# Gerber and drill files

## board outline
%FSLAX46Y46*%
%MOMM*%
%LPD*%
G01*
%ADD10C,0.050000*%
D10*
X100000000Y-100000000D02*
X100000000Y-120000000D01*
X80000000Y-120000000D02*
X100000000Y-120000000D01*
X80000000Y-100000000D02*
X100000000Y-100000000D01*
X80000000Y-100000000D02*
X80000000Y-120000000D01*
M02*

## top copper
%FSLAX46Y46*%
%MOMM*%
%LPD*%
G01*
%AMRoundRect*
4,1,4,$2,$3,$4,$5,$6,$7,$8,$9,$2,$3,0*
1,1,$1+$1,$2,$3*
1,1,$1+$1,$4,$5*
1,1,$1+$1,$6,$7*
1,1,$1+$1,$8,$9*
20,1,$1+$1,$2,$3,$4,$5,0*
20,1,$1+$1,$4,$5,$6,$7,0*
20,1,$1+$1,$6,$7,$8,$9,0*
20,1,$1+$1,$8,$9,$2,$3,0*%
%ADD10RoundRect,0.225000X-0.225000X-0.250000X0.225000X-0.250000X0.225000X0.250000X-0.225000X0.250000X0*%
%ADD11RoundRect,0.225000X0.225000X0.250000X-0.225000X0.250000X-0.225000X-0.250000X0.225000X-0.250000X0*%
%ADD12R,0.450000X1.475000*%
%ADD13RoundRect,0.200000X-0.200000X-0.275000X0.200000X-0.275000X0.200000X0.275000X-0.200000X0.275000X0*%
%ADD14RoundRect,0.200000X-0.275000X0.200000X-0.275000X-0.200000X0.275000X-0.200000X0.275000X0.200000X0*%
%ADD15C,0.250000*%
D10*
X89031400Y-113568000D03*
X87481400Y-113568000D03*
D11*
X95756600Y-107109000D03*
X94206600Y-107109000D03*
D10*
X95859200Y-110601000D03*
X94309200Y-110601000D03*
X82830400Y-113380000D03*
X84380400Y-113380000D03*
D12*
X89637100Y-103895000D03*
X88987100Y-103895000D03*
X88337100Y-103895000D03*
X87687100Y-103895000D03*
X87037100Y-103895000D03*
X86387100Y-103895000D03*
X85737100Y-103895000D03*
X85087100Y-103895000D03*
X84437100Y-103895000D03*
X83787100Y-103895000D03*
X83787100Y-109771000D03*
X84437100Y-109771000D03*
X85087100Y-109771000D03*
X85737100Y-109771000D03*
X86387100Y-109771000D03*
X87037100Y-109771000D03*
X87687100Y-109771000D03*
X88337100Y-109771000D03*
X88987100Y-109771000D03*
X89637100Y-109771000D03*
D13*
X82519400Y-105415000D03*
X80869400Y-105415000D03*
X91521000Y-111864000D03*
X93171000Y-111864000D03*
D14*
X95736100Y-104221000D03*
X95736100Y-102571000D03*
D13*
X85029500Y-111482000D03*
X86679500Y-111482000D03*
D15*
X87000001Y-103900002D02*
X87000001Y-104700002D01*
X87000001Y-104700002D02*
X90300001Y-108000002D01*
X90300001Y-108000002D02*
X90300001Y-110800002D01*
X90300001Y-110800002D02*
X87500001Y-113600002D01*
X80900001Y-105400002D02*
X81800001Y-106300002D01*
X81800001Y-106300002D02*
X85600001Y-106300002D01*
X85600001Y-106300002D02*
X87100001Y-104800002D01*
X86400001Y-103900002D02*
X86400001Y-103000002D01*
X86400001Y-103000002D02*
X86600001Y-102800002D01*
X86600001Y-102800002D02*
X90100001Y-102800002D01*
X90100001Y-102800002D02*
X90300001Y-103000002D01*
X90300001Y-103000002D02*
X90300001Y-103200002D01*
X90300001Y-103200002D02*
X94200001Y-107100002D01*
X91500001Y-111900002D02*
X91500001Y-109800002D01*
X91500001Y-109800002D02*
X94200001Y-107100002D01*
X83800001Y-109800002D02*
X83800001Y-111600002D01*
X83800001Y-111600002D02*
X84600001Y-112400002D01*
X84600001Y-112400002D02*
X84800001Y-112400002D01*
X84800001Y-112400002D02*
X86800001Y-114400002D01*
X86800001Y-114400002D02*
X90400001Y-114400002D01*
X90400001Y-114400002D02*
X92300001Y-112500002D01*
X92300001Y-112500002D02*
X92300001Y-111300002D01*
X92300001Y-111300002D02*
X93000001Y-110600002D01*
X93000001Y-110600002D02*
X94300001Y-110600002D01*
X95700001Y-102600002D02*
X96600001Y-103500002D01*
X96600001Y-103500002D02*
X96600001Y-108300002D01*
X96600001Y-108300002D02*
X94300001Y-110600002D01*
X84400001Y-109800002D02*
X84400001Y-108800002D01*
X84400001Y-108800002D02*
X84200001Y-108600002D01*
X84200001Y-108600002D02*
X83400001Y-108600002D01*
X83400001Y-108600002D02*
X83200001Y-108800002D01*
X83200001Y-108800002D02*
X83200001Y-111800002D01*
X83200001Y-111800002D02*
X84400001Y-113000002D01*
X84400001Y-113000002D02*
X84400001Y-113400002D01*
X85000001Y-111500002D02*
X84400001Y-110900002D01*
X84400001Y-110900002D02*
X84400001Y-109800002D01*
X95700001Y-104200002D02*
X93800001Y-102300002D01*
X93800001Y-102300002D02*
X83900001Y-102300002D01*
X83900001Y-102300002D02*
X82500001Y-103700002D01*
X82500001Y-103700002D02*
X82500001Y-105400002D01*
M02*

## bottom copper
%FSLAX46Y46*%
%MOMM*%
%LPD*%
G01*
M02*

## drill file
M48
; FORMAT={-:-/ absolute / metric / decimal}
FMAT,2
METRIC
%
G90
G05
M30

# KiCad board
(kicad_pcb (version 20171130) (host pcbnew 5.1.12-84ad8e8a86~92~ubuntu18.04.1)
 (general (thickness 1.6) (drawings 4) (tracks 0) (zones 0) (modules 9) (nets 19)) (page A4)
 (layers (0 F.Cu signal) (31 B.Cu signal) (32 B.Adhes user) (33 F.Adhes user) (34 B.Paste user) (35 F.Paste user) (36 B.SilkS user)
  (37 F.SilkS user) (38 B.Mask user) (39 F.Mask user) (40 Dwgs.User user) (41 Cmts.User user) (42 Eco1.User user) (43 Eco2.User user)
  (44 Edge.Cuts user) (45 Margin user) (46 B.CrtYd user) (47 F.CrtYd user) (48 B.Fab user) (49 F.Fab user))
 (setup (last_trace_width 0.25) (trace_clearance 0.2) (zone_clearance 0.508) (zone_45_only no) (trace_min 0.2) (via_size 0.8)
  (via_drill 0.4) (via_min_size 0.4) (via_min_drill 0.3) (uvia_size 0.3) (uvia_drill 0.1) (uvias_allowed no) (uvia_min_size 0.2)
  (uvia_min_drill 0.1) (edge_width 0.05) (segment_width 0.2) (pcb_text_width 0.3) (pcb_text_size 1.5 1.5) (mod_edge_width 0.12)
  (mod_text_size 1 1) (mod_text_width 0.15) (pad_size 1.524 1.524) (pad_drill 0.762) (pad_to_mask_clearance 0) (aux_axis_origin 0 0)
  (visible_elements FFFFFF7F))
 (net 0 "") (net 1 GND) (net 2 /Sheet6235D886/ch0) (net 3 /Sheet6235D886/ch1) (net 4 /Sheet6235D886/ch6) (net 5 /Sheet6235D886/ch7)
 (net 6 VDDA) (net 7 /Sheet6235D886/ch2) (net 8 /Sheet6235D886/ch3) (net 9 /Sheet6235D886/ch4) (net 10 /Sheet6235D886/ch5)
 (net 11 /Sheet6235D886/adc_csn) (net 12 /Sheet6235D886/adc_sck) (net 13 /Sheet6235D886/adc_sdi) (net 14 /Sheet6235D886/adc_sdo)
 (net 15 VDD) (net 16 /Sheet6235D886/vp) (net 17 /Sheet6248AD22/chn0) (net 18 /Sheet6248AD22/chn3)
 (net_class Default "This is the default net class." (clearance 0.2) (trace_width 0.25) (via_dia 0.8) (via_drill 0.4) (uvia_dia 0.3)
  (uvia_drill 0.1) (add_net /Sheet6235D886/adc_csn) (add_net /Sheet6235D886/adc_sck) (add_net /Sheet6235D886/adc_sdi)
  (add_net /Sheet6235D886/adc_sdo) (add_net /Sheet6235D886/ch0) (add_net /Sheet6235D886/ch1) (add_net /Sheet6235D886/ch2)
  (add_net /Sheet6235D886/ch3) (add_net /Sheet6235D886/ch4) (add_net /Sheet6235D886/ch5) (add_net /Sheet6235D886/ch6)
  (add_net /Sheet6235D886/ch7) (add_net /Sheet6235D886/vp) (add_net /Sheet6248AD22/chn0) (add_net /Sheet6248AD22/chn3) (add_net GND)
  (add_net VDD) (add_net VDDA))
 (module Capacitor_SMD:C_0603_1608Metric (layer F.Cu) (at 88.256400 113.568000)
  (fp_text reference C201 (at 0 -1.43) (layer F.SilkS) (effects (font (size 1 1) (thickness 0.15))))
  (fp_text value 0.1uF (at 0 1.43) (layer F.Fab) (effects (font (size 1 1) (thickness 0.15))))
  (pad 2 smd roundrect (at 0.775 0) (size 0.9 0.95) (layers F.Cu F.Mask F.Paste) (roundrect_rratio 0.25) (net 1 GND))
  (pad 1 smd roundrect (at -0.775 0) (size 0.9 0.95) (layers F.Cu F.Mask F.Paste) (roundrect_rratio 0.25) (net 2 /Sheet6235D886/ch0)))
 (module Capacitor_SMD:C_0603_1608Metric (layer F.Cu) (at 94.981600 107.109000 180.000000)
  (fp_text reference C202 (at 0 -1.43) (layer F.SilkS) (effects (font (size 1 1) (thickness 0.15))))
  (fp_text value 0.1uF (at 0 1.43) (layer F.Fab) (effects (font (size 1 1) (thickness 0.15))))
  (pad 1 smd roundrect (at -0.775 0 180.000000) (size 0.9 0.95) (layers F.Cu F.Mask F.Paste) (roundrect_rratio 0.25) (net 1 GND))
  (pad 2 smd roundrect (at 0.775 0 180.000000) (size 0.9 0.95) (layers F.Cu F.Mask F.Paste) (roundrect_rratio 0.25)
   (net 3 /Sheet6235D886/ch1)))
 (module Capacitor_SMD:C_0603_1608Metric (layer F.Cu) (at 95.084200 110.601000)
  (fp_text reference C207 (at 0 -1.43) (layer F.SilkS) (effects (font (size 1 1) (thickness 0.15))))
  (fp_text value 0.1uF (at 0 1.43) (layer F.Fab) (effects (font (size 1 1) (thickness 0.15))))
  (pad 2 smd roundrect (at 0.775 0) (size 0.9 0.95) (layers F.Cu F.Mask F.Paste) (roundrect_rratio 0.25) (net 1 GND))
  (pad 1 smd roundrect (at -0.775 0) (size 0.9 0.95) (layers F.Cu F.Mask F.Paste) (roundrect_rratio 0.25) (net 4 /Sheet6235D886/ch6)))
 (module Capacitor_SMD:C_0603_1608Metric (layer F.Cu) (at 83.605400 113.380000)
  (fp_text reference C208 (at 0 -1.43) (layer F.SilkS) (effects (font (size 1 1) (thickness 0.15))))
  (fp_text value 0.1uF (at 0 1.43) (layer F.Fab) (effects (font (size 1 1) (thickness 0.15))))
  (pad 1 smd roundrect (at -0.775 0) (size 0.9 0.95) (layers F.Cu F.Mask F.Paste) (roundrect_rratio 0.25) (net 1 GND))
  (pad 2 smd roundrect (at 0.775 0) (size 0.9 0.95) (layers F.Cu F.Mask F.Paste) (roundrect_rratio 0.25) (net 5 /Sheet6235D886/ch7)))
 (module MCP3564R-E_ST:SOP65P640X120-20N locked (layer F.Cu) (at 86.712100 106.833000 270.000000)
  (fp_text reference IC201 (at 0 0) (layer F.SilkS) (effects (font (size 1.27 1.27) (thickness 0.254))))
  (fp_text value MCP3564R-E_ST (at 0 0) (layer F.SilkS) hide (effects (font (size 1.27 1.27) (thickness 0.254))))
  (pad 1 smd rect (at -2.938 -2.925) (size 0.45 1.475) (layers F.Cu F.Mask F.Paste) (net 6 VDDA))
  (pad 2 smd rect (at -2.938 -2.275) (size 0.45 1.475) (layers F.Cu F.Mask F.Paste) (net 1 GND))
  (pad 3 smd rect (at -2.938 -1.625) (size 0.45 1.475) (layers F.Cu F.Mask F.Paste) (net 1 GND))
  (pad 4 smd rect (at -2.938 -0.975) (size 0.45 1.475) (layers F.Cu F.Mask F.Paste))
  (pad 5 smd rect (at -2.938 -0.325) (size 0.45 1.475) (layers F.Cu F.Mask F.Paste) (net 2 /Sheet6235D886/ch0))
  (pad 6 smd rect (at -2.938 0.325) (size 0.45 1.475) (layers F.Cu F.Mask F.Paste) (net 3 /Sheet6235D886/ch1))
  (pad 7 smd rect (at -2.938 0.975) (size 0.45 1.475) (layers F.Cu F.Mask F.Paste) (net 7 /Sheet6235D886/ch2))
  (pad 8 smd rect (at -2.938 1.625) (size 0.45 1.475) (layers F.Cu F.Mask F.Paste) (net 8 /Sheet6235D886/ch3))
  (pad 9 smd rect (at -2.938 2.275) (size 0.45 1.475) (layers F.Cu F.Mask F.Paste) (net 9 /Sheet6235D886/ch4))
  (pad 10 smd rect (at -2.938 2.925) (size 0.45 1.475) (layers F.Cu F.Mask F.Paste) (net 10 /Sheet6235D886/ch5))
  (pad 11 smd rect (at 2.938 2.925) (size 0.45 1.475) (layers F.Cu F.Mask F.Paste) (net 4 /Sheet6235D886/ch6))
  (pad 12 smd rect (at 2.938 2.275) (size 0.45 1.475) (layers F.Cu F.Mask F.Paste) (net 5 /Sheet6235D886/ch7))
  (pad 13 smd rect (at 2.938 1.625) (size 0.45 1.475) (layers F.Cu F.Mask F.Paste) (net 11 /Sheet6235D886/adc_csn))
  (pad 14 smd rect (at 2.938 0.975) (size 0.45 1.475) (layers F.Cu F.Mask F.Paste) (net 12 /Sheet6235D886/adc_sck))
  (pad 15 smd rect (at 2.938 0.325) (size 0.45 1.475) (layers F.Cu F.Mask F.Paste) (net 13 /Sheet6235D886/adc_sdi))
  (pad 16 smd rect (at 2.938 -0.325) (size 0.45 1.475) (layers F.Cu F.Mask F.Paste) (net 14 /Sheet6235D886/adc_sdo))
  (pad 17 smd rect (at 2.938 -0.975) (size 0.45 1.475) (layers F.Cu F.Mask F.Paste))
  (pad 18 smd rect (at 2.938 -1.625) (size 0.45 1.475) (layers F.Cu F.Mask F.Paste))
  (pad 19 smd rect (at 2.938 -2.275) (size 0.45 1.475) (layers F.Cu F.Mask F.Paste) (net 1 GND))
  (pad 20 smd rect (at 2.938 -2.925) (size 0.45 1.475) (layers F.Cu F.Mask F.Paste) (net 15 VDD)))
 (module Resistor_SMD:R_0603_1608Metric (layer F.Cu) (at 81.694400 105.415000)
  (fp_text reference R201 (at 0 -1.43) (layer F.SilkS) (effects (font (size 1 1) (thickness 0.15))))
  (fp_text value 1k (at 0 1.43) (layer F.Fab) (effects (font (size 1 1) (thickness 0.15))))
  (pad 2 smd roundrect (at 0.825 0) (size 0.8 0.95) (layers F.Cu F.Mask F.Paste) (roundrect_rratio 0.25) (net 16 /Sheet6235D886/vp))
  (pad 1 smd roundrect (at -0.825 0) (size 0.8 0.95) (layers F.Cu F.Mask F.Paste) (roundrect_rratio 0.25) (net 2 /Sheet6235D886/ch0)))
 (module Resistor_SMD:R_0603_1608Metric (layer F.Cu) (at 92.346000 111.864000)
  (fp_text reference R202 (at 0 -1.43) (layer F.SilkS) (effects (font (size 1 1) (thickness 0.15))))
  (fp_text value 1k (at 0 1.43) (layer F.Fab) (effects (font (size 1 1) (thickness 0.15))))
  (pad 1 smd roundrect (at -0.825 0) (size 0.8 0.95) (layers F.Cu F.Mask F.Paste) (roundrect_rratio 0.25) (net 3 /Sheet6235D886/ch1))
  (pad 2 smd roundrect (at 0.825 0) (size 0.8 0.95) (layers F.Cu F.Mask F.Paste) (roundrect_rratio 0.25) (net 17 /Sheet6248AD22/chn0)))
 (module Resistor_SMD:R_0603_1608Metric (layer F.Cu) (at 95.736100 103.396000 270.000000)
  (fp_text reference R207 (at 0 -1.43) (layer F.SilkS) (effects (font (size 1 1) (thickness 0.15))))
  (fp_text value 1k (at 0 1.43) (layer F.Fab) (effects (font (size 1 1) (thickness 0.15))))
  (pad 2 smd roundrect (at 0.825 0 270.000000) (size 0.8 0.95) (layers F.Cu F.Mask F.Paste) (roundrect_rratio 0.25)
   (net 16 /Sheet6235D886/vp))
  (pad 1 smd roundrect (at -0.825 0 270.000000) (size 0.8 0.95) (layers F.Cu F.Mask F.Paste) (roundrect_rratio 0.25)
   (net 4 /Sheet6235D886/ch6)))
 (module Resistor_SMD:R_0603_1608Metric (layer F.Cu) (at 85.854500 111.482000)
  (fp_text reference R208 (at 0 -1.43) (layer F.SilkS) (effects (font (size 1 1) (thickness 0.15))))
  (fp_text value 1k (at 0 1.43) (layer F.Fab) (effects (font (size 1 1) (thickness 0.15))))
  (pad 1 smd roundrect (at -0.825 0) (size 0.8 0.95) (layers F.Cu F.Mask F.Paste) (roundrect_rratio 0.25) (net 5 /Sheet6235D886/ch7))
  (pad 2 smd roundrect (at 0.825 0) (size 0.8 0.95) (layers F.Cu F.Mask F.Paste) (roundrect_rratio 0.25) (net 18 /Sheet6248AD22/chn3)))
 (gr_line (start 100 100) (end 100 120) (layer Edge.Cuts) (width 0.05))
 (gr_line (start 80 120) (end 100 120) (layer Edge.Cuts) (width 0.05))
 (gr_line (start 80 100) (end 100 100) (layer Edge.Cuts) (width 0.05))
 (gr_line (start 80 100) (end 80 120) (layer Edge.Cuts) (width 0.05))
 (segment (start 87.000001 103.900002) (end 87.000001 104.700002) (width 0.250000) (layer F.Cu) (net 2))
 (segment (start 87.000001 104.700002) (end 90.300001 108.000002) (width 0.250000) (layer F.Cu) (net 2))
 (segment (start 90.300001 108.000002) (end 90.300001 110.800002) (width 0.250000) (layer F.Cu) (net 2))
 (segment (start 90.300001 110.800002) (end 87.500001 113.600002) (width 0.250000) (layer F.Cu) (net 2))
 (segment (start 80.900001 105.400002) (end 81.800001 106.300002) (width 0.250000) (layer F.Cu) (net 2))
 (segment (start 81.800001 106.300002) (end 85.600001 106.300002) (width 0.250000) (layer F.Cu) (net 2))
 (segment (start 85.600001 106.300002) (end 87.100001 104.800002) (width 0.250000) (layer F.Cu) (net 2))
 (segment (start 86.400001 103.900002) (end 86.400001 103.000002) (width 0.250000) (layer F.Cu) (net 3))
 (segment (start 86.400001 103.000002) (end 86.600001 102.800002) (width 0.250000) (layer F.Cu) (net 3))
 (segment (start 86.600001 102.800002) (end 90.100001 102.800002) (width 0.250000) (layer F.Cu) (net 3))
 (segment (start 90.100001 102.800002) (end 90.300001 103.000002) (width 0.250000) (layer F.Cu) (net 3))
 (segment (start 90.300001 103.000002) (end 90.300001 103.200002) (width 0.250000) (layer F.Cu) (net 3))
 (segment (start 90.300001 103.200002) (end 94.200001 107.100002) (width 0.250000) (layer F.Cu) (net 3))
 (segment (start 91.500001 111.900002) (end 91.500001 109.800002) (width 0.250000) (layer F.Cu) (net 3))
 (segment (start 91.500001 109.800002) (end 94.200001 107.100002) (width 0.250000) (layer F.Cu) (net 3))
 (segment (start 83.800001 109.800002) (end 83.800001 111.600002) (width 0.250000) (layer F.Cu) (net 4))
 (segment (start 83.800001 111.600002) (end 84.600001 112.400002) (width 0.250000) (layer F.Cu) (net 4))
 (segment (start 84.600001 112.400002) (end 84.800001 112.400002) (width 0.250000) (layer F.Cu) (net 4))
 (segment (start 84.800001 112.400002) (end 86.800001 114.400002) (width 0.250000) (layer F.Cu) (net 4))
 (segment (start 86.800001 114.400002) (end 90.400001 114.400002) (width 0.250000) (layer F.Cu) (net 4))
 (segment (start 90.400001 114.400002) (end 92.300001 112.500002) (width 0.250000) (layer F.Cu) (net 4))
 (segment (start 92.300001 112.500002) (end 92.300001 111.300002) (width 0.250000) (layer F.Cu) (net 4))
 (segment (start 92.300001 111.300002) (end 93.000001 110.600002) (width 0.250000) (layer F.Cu) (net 4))
 (segment (start 93.000001 110.600002) (end 94.300001 110.600002) (width 0.250000) (layer F.Cu) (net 4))
 (segment (start 95.700001 102.600002) (end 96.600001 103.500002) (width 0.250000) (layer F.Cu) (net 4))
 (segment (start 96.600001 103.500002) (end 96.600001 108.300002) (width 0.250000) (layer F.Cu) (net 4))
 (segment (start 96.600001 108.300002) (end 94.300001 110.600002) (width 0.250000) (layer F.Cu) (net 4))
 (segment (start 84.400001 109.800002) (end 84.400001 108.800002) (width 0.250000) (layer F.Cu) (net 5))
 (segment (start 84.400001 108.800002) (end 84.200001 108.600002) (width 0.250000) (layer F.Cu) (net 5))
 (segment (start 84.200001 108.600002) (end 83.400001 108.600002) (width 0.250000) (layer F.Cu) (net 5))
 (segment (start 83.400001 108.600002) (end 83.200001 108.800002) (width 0.250000) (layer F.Cu) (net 5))
 (segment (start 83.200001 108.800002) (end 83.200001 111.800002) (width 0.250000) (layer F.Cu) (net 5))
 (segment (start 83.200001 111.800002) (end 84.400001 113.000002) (width 0.250000) (layer F.Cu) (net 5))
 (segment (start 84.400001 113.000002) (end 84.400001 113.400002) (width 0.250000) (layer F.Cu) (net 5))
 (segment (start 85.000001 111.500002) (end 84.400001 110.900002) (width 0.250000) (layer F.Cu) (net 5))
 (segment (start 84.400001 110.900002) (end 84.400001 109.800002) (width 0.250000) (layer F.Cu) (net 5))
 (segment (start 95.700001 104.200002) (end 93.800001 102.300002) (width 0.250000) (layer F.Cu) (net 16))
 (segment (start 93.800001 102.300002) (end 83.900001 102.300002) (width 0.250000) (layer F.Cu) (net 16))
 (segment (start 83.900001 102.300002) (end 82.500001 103.700002) (width 0.250000) (layer F.Cu) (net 16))
 (segment (start 82.500001 103.700002) (end 82.500001 105.400002) (width 0.250000) (layer F.Cu) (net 16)))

